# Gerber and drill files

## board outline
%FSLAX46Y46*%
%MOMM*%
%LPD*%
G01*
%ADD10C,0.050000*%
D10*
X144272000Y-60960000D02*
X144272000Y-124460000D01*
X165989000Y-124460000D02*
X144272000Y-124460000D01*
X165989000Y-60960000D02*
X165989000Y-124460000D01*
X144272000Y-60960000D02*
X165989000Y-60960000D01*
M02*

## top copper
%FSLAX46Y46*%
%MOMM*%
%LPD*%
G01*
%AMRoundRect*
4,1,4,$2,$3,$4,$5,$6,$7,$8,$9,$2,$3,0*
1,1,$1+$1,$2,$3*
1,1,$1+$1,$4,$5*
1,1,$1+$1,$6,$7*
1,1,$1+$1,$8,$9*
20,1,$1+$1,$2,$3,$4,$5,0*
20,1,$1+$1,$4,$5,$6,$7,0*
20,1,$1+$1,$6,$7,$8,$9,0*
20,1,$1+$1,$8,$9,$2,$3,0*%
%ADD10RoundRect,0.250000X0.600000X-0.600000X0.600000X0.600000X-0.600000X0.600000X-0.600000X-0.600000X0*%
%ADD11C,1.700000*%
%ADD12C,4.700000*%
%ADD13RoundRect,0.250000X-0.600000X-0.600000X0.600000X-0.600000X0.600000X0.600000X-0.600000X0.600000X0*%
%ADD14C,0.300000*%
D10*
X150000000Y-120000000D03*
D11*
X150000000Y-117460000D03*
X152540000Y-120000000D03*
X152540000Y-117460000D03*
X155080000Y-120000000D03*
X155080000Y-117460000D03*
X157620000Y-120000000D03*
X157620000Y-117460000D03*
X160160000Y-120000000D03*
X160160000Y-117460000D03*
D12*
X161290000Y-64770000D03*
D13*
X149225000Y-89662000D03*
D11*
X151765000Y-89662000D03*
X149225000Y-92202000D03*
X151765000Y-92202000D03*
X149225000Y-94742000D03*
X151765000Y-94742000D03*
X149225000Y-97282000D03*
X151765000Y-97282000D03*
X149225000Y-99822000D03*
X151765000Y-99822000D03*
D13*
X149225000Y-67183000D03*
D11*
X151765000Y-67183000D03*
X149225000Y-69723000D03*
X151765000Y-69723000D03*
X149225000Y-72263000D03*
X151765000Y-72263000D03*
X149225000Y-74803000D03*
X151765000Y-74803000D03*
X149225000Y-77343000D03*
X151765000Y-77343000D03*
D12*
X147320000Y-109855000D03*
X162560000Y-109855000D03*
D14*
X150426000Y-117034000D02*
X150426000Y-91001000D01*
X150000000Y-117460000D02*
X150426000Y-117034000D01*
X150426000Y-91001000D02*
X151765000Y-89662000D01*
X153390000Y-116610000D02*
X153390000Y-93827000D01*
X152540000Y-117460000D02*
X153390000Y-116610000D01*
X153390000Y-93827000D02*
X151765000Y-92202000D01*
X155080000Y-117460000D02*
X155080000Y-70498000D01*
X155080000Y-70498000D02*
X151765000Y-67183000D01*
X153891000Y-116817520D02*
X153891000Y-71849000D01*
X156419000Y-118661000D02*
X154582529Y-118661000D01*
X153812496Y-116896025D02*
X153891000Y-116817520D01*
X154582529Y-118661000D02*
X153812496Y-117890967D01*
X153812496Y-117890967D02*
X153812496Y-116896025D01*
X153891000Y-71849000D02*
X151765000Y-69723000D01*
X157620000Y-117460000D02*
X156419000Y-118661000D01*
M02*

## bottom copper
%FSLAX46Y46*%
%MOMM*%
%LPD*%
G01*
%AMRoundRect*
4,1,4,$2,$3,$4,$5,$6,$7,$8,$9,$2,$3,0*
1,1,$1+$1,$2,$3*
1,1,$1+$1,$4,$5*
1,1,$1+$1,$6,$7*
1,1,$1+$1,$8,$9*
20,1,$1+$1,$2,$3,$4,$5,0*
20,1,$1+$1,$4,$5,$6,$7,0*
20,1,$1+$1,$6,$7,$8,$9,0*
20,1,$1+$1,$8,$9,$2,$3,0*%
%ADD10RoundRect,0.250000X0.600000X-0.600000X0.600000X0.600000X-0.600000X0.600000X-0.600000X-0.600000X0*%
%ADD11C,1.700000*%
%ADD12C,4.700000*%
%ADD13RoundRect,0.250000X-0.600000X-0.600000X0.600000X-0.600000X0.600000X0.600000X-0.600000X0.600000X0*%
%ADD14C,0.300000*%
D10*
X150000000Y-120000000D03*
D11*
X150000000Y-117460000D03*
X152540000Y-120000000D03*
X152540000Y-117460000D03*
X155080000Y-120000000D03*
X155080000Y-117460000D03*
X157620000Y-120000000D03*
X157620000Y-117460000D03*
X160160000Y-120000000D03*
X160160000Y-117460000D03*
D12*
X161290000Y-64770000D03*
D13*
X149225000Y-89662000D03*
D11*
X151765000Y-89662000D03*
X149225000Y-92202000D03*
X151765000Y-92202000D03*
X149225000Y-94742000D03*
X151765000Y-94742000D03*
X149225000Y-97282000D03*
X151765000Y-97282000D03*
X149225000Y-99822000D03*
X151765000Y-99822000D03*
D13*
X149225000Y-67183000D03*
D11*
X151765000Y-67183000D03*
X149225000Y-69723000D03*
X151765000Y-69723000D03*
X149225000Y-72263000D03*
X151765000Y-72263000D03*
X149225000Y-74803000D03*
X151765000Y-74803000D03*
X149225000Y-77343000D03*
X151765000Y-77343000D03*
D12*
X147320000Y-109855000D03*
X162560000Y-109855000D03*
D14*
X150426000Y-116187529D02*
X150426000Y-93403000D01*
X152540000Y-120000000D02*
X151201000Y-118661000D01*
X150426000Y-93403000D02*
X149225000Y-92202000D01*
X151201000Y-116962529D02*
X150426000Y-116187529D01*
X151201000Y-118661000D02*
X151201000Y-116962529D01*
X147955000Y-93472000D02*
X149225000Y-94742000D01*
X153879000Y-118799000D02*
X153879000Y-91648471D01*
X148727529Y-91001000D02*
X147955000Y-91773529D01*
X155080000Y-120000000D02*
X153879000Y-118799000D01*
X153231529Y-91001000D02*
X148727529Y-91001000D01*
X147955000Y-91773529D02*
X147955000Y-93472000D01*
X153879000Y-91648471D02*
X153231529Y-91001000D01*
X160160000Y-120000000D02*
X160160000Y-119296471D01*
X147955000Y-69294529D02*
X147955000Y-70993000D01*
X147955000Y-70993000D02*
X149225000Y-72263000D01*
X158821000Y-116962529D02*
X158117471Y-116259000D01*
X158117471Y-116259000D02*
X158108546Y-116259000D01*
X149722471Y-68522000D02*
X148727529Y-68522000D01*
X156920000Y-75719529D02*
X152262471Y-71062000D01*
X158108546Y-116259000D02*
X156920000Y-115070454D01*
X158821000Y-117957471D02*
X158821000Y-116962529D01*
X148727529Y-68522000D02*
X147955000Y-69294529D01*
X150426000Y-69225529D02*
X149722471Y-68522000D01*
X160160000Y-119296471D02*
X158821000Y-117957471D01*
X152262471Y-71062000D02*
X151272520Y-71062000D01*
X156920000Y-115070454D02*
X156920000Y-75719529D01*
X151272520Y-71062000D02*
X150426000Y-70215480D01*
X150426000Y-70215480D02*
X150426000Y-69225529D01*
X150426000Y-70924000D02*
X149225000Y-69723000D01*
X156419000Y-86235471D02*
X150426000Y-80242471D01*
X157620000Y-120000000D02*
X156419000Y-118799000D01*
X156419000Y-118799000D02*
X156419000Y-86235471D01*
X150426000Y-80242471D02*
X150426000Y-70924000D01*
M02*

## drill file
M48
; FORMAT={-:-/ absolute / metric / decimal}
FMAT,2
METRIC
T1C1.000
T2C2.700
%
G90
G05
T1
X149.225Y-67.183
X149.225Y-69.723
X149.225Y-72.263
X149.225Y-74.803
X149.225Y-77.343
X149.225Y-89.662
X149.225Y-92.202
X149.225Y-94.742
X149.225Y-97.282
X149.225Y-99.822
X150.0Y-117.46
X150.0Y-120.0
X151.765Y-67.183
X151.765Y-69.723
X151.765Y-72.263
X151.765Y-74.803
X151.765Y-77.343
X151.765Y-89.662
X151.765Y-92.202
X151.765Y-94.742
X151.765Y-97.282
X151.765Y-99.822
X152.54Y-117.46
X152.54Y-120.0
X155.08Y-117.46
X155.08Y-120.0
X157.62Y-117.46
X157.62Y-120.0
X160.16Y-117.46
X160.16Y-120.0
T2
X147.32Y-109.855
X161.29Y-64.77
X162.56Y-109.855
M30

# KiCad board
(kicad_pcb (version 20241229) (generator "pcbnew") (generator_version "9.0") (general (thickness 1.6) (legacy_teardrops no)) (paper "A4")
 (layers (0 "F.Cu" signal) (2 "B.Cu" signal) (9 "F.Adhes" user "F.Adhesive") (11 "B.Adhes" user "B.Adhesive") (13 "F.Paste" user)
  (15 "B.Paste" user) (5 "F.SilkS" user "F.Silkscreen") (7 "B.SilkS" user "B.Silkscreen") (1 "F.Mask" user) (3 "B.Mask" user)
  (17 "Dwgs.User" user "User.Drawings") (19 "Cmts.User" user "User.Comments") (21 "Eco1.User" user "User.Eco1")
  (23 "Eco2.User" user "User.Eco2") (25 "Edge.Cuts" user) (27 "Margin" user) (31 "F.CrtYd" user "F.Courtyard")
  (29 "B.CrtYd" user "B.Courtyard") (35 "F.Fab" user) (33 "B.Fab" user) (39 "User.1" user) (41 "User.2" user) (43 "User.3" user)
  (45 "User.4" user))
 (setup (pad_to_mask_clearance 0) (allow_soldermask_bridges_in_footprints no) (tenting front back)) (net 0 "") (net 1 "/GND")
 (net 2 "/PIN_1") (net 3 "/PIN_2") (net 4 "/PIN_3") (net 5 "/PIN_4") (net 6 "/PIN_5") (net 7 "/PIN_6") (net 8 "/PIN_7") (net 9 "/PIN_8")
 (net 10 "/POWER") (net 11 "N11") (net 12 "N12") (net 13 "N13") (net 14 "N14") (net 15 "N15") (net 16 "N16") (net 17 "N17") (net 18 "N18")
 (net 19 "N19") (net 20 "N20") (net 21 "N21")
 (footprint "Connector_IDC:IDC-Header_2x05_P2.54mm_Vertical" (layer "F.Cu") (at 150 120 90)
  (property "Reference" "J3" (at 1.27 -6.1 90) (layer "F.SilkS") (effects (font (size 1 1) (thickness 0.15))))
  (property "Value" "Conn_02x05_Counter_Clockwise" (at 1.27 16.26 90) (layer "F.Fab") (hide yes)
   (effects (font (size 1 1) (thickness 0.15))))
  (pad "1" thru_hole roundrect (at 0 0 90) (size 1.7 1.7) (drill 1) (layers "*.Cu" "*.Mask") (remove_unused_layers no)
   (roundrect_rratio 0.147059) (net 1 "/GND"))
  (pad "2" thru_hole circle (at 2.54 0 90) (size 1.7 1.7) (drill 1) (layers "*.Cu" "*.Mask") (remove_unused_layers no) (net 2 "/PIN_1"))
  (pad "3" thru_hole circle (at 0 2.54 90) (size 1.7 1.7) (drill 1) (layers "*.Cu" "*.Mask") (remove_unused_layers no) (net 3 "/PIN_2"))
  (pad "4" thru_hole circle (at 2.54 2.54 90) (size 1.7 1.7) (drill 1) (layers "*.Cu" "*.Mask") (remove_unused_layers no) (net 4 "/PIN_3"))
  (pad "5" thru_hole circle (at 0 5.08 90) (size 1.7 1.7) (drill 1) (layers "*.Cu" "*.Mask") (remove_unused_layers no) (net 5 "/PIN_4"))
  (pad "6" thru_hole circle (at 2.54 5.08 90) (size 1.7 1.7) (drill 1) (layers "*.Cu" "*.Mask") (remove_unused_layers no) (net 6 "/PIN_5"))
  (pad "7" thru_hole circle (at 0 7.62 90) (size 1.7 1.7) (drill 1) (layers "*.Cu" "*.Mask") (remove_unused_layers no) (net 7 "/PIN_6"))
  (pad "8" thru_hole circle (at 2.54 7.62 90) (size 1.7 1.7) (drill 1) (layers "*.Cu" "*.Mask") (remove_unused_layers no) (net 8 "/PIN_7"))
  (pad "9" thru_hole circle (at 0 10.16 90) (size 1.7 1.7) (drill 1) (layers "*.Cu" "*.Mask") (remove_unused_layers no) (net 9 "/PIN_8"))
  (pad "10" thru_hole circle (at 2.54 10.16 90) (size 1.7 1.7) (drill 1) (layers "*.Cu" "*.Mask") (remove_unused_layers no)
   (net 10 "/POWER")))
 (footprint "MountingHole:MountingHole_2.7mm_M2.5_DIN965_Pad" (layer "F.Cu") (at 161.29 64.77)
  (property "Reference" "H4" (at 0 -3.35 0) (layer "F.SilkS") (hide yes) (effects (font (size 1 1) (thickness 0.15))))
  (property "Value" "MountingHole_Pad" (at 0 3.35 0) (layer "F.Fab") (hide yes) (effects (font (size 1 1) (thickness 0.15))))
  (pad "1" thru_hole circle (at 0 0) (size 4.7 4.7) (drill 2.7) (layers "*.Cu" "*.Mask") (remove_unused_layers no) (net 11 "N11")))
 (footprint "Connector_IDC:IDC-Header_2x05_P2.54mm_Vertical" (layer "F.Cu") (at 149.225 89.662)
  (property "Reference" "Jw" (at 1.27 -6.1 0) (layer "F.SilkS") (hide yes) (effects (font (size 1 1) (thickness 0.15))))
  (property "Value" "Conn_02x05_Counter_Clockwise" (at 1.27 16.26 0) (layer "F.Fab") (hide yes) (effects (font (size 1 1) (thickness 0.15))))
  (pad "1" thru_hole roundrect (at 0 0) (size 1.7 1.7) (drill 1) (layers "*.Cu" "*.Mask") (remove_unused_layers no)
   (roundrect_rratio 0.147059) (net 1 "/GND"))
  (pad "2" thru_hole circle (at 2.54 0) (size 1.7 1.7) (drill 1) (layers "*.Cu" "*.Mask") (remove_unused_layers no) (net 2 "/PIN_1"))
  (pad "3" thru_hole circle (at 0 2.54) (size 1.7 1.7) (drill 1) (layers "*.Cu" "*.Mask") (remove_unused_layers no) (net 3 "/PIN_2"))
  (pad "4" thru_hole circle (at 2.54 2.54) (size 1.7 1.7) (drill 1) (layers "*.Cu" "*.Mask") (remove_unused_layers no) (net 4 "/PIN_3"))
  (pad "5" thru_hole circle (at 0 5.08) (size 1.7 1.7) (drill 1) (layers "*.Cu" "*.Mask") (remove_unused_layers no) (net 5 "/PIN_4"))
  (pad "6" thru_hole circle (at 2.54 5.08) (size 1.7 1.7) (drill 1) (layers "*.Cu" "*.Mask") (remove_unused_layers no) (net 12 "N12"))
  (pad "7" thru_hole circle (at 0 7.62) (size 1.7 1.7) (drill 1) (layers "*.Cu" "*.Mask") (remove_unused_layers no) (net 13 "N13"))
  (pad "8" thru_hole circle (at 2.54 7.62) (size 1.7 1.7) (drill 1) (layers "*.Cu" "*.Mask") (remove_unused_layers no) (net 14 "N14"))
  (pad "9" thru_hole circle (at 0 10.16) (size 1.7 1.7) (drill 1) (layers "*.Cu" "*.Mask") (remove_unused_layers no) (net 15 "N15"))
  (pad "10" thru_hole circle (at 2.54 10.16) (size 1.7 1.7) (drill 1) (layers "*.Cu" "*.Mask") (remove_unused_layers no) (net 10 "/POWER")))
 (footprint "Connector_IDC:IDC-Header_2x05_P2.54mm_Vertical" (layer "F.Cu") (at 149.225 67.183)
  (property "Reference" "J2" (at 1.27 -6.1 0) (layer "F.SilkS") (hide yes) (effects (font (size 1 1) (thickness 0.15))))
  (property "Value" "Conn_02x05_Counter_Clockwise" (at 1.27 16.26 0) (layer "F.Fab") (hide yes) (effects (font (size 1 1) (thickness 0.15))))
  (pad "1" thru_hole roundrect (at 0 0) (size 1.7 1.7) (drill 1) (layers "*.Cu" "*.Mask") (remove_unused_layers no)
   (roundrect_rratio 0.147059) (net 1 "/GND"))
  (pad "2" thru_hole circle (at 2.54 0) (size 1.7 1.7) (drill 1) (layers "*.Cu" "*.Mask") (remove_unused_layers no) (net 6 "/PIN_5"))
  (pad "3" thru_hole circle (at 0 2.54) (size 1.7 1.7) (drill 1) (layers "*.Cu" "*.Mask") (remove_unused_layers no) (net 7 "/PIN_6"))
  (pad "4" thru_hole circle (at 2.54 2.54) (size 1.7 1.7) (drill 1) (layers "*.Cu" "*.Mask") (remove_unused_layers no) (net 8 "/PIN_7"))
  (pad "5" thru_hole circle (at 0 5.08) (size 1.7 1.7) (drill 1) (layers "*.Cu" "*.Mask") (remove_unused_layers no) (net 9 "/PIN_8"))
  (pad "6" thru_hole circle (at 2.54 5.08) (size 1.7 1.7) (drill 1) (layers "*.Cu" "*.Mask") (remove_unused_layers no) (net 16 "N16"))
  (pad "7" thru_hole circle (at 0 7.62) (size 1.7 1.7) (drill 1) (layers "*.Cu" "*.Mask") (remove_unused_layers no) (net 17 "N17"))
  (pad "8" thru_hole circle (at 2.54 7.62) (size 1.7 1.7) (drill 1) (layers "*.Cu" "*.Mask") (remove_unused_layers no) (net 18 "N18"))
  (pad "9" thru_hole circle (at 0 10.16) (size 1.7 1.7) (drill 1) (layers "*.Cu" "*.Mask") (remove_unused_layers no) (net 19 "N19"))
  (pad "10" thru_hole circle (at 2.54 10.16) (size 1.7 1.7) (drill 1) (layers "*.Cu" "*.Mask") (remove_unused_layers no) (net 10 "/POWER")))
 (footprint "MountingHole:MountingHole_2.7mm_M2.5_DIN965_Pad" (layer "F.Cu") (at 147.32 109.855)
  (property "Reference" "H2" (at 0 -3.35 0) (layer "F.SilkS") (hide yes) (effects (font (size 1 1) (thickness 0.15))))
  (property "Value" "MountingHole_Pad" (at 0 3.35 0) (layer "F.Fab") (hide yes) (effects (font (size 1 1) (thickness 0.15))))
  (pad "1" thru_hole circle (at 0 0) (size 4.7 4.7) (drill 2.7) (layers "*.Cu" "*.Mask") (remove_unused_layers no) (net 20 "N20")))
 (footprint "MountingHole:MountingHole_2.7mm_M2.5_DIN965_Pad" (layer "F.Cu") (at 162.56 109.855)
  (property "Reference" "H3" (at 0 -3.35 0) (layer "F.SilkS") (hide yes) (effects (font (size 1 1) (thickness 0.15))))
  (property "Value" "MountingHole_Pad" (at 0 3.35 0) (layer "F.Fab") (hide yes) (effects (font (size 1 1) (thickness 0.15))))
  (pad "1" thru_hole circle (at 0 0) (size 4.7 4.7) (drill 2.7) (layers "*.Cu" "*.Mask") (remove_unused_layers no) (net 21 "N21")))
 (gr_line (start 144.272 60.96) (end 144.272 124.46) (stroke (width 0.05) (type default)) (layer "Edge.Cuts"))
 (gr_line (start 165.989 124.46) (end 144.272 124.46) (stroke (width 0.05) (type default)) (layer "Edge.Cuts"))
 (gr_line (start 165.989 60.96) (end 165.989 124.46) (stroke (width 0.05) (type default)) (layer "Edge.Cuts"))
 (gr_line (start 144.272 60.96) (end 165.989 60.96) (stroke (width 0.05) (type default)) (layer "Edge.Cuts"))
 (segment (start 150.426 117.034) (end 150.426 91.001) (width 0.3) (layer "F.Cu") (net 2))
 (segment (start 150 117.46) (end 150.426 117.034) (width 0.3) (layer "F.Cu") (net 2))
 (segment (start 150.426 91.001) (end 151.765 89.662) (width 0.3) (layer "F.Cu") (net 2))
 (segment (start 150.426 116.187529) (end 150.426 93.403) (width 0.3) (layer "B.Cu") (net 3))
 (segment (start 152.54 120) (end 151.201 118.661) (width 0.3) (layer "B.Cu") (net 3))
 (segment (start 150.426 93.403) (end 149.225 92.202) (width 0.3) (layer "B.Cu") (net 3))
 (segment (start 151.201 116.962529) (end 150.426 116.187529) (width 0.3) (layer "B.Cu") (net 3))
 (segment (start 151.201 118.661) (end 151.201 116.962529) (width 0.3) (layer "B.Cu") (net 3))
 (segment (start 147.955 93.472) (end 149.225 94.742) (width 0.3) (layer "B.Cu") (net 5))
 (segment (start 153.879 118.799) (end 153.879 91.648471) (width 0.3) (layer "B.Cu") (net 5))
 (segment (start 148.727529 91.001) (end 147.955 91.773529) (width 0.3) (layer "B.Cu") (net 5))
 (segment (start 155.08 120) (end 153.879 118.799) (width 0.3) (layer "B.Cu") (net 5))
 (segment (start 153.231529 91.001) (end 148.727529 91.001) (width 0.3) (layer "B.Cu") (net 5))
 (segment (start 147.955 91.773529) (end 147.955 93.472) (width 0.3) (layer "B.Cu") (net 5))
 (segment (start 153.879 91.648471) (end 153.231529 91.001) (width 0.3) (layer "B.Cu") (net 5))
 (segment (start 153.39 116.61) (end 153.39 93.827) (width 0.3) (layer "F.Cu") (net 4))
 (segment (start 152.54 117.46) (end 153.39 116.61) (width 0.3) (layer "F.Cu") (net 4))
 (segment (start 153.39 93.827) (end 151.765 92.202) (width 0.3) (layer "F.Cu") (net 4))
 (segment (start 155.08 117.46) (end 155.08 70.498) (width 0.3) (layer "F.Cu") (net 6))
 (segment (start 155.08 70.498) (end 151.765 67.183) (width 0.3) (layer "F.Cu") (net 6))
 (segment (start 160.16 120) (end 160.16 119.296471) (width 0.3) (layer "B.Cu") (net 9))
 (segment (start 147.955 69.294529) (end 147.955 70.993) (width 0.3) (layer "B.Cu") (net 9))
 (segment (start 147.955 70.993) (end 149.225 72.263) (width 0.3) (layer "B.Cu") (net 9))
 (segment (start 158.821 116.962529) (end 158.117471 116.259) (width 0.3) (layer "B.Cu") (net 9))
 (segment (start 158.117471 116.259) (end 158.108546 116.259) (width 0.3) (layer "B.Cu") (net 9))
 (segment (start 149.722471 68.522) (end 148.727529 68.522) (width 0.3) (layer "B.Cu") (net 9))
 (segment (start 156.92 75.719529) (end 152.262471 71.062) (width 0.3) (layer "B.Cu") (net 9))
 (segment (start 158.108546 116.259) (end 156.92 115.070454) (width 0.3) (layer "B.Cu") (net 9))
 (segment (start 158.821 117.957471) (end 158.821 116.962529) (width 0.3) (layer "B.Cu") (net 9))
 (segment (start 148.727529 68.522) (end 147.955 69.294529) (width 0.3) (layer "B.Cu") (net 9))
 (segment (start 150.426 69.225529) (end 149.722471 68.522) (width 0.3) (layer "B.Cu") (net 9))
 (segment (start 160.16 119.296471) (end 158.821 117.957471) (width 0.3) (layer "B.Cu") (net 9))
 (segment (start 152.262471 71.062) (end 151.27252 71.062) (width 0.3) (layer "B.Cu") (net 9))
 (segment (start 156.92 115.070454) (end 156.92 75.719529) (width 0.3) (layer "B.Cu") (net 9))
 (segment (start 151.27252 71.062) (end 150.426 70.21548) (width 0.3) (layer "B.Cu") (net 9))
 (segment (start 150.426 70.21548) (end 150.426 69.225529) (width 0.3) (layer "B.Cu") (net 9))
 (segment (start 153.891 116.81752) (end 153.891 71.849) (width 0.3) (layer "F.Cu") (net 8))
 (segment (start 156.419 118.661) (end 154.582529 118.661) (width 0.3) (layer "F.Cu") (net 8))
 (segment (start 153.812496 116.896025) (end 153.891 116.81752) (width 0.3) (layer "F.Cu") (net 8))
 (segment (start 154.582529 118.661) (end 153.812496 117.890967) (width 0.3) (layer "F.Cu") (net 8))
 (segment (start 153.812496 117.890967) (end 153.812496 116.896025) (width 0.3) (layer "F.Cu") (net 8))
 (segment (start 153.891 71.849) (end 151.765 69.723) (width 0.3) (layer "F.Cu") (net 8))
 (segment (start 157.62 117.46) (end 156.419 118.661) (width 0.3) (layer "F.Cu") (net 8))
 (segment (start 150.426 70.924) (end 149.225 69.723) (width 0.3) (layer "B.Cu") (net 7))
 (segment (start 156.419 86.235471) (end 150.426 80.242471) (width 0.3) (layer "B.Cu") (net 7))
 (segment (start 157.62 120) (end 156.419 118.799) (width 0.3) (layer "B.Cu") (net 7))
 (segment (start 156.419 118.799) (end 156.419 86.235471) (width 0.3) (layer "B.Cu") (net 7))
 (segment (start 150.426 80.242471) (end 150.426 70.924) (width 0.3) (layer "B.Cu") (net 7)))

